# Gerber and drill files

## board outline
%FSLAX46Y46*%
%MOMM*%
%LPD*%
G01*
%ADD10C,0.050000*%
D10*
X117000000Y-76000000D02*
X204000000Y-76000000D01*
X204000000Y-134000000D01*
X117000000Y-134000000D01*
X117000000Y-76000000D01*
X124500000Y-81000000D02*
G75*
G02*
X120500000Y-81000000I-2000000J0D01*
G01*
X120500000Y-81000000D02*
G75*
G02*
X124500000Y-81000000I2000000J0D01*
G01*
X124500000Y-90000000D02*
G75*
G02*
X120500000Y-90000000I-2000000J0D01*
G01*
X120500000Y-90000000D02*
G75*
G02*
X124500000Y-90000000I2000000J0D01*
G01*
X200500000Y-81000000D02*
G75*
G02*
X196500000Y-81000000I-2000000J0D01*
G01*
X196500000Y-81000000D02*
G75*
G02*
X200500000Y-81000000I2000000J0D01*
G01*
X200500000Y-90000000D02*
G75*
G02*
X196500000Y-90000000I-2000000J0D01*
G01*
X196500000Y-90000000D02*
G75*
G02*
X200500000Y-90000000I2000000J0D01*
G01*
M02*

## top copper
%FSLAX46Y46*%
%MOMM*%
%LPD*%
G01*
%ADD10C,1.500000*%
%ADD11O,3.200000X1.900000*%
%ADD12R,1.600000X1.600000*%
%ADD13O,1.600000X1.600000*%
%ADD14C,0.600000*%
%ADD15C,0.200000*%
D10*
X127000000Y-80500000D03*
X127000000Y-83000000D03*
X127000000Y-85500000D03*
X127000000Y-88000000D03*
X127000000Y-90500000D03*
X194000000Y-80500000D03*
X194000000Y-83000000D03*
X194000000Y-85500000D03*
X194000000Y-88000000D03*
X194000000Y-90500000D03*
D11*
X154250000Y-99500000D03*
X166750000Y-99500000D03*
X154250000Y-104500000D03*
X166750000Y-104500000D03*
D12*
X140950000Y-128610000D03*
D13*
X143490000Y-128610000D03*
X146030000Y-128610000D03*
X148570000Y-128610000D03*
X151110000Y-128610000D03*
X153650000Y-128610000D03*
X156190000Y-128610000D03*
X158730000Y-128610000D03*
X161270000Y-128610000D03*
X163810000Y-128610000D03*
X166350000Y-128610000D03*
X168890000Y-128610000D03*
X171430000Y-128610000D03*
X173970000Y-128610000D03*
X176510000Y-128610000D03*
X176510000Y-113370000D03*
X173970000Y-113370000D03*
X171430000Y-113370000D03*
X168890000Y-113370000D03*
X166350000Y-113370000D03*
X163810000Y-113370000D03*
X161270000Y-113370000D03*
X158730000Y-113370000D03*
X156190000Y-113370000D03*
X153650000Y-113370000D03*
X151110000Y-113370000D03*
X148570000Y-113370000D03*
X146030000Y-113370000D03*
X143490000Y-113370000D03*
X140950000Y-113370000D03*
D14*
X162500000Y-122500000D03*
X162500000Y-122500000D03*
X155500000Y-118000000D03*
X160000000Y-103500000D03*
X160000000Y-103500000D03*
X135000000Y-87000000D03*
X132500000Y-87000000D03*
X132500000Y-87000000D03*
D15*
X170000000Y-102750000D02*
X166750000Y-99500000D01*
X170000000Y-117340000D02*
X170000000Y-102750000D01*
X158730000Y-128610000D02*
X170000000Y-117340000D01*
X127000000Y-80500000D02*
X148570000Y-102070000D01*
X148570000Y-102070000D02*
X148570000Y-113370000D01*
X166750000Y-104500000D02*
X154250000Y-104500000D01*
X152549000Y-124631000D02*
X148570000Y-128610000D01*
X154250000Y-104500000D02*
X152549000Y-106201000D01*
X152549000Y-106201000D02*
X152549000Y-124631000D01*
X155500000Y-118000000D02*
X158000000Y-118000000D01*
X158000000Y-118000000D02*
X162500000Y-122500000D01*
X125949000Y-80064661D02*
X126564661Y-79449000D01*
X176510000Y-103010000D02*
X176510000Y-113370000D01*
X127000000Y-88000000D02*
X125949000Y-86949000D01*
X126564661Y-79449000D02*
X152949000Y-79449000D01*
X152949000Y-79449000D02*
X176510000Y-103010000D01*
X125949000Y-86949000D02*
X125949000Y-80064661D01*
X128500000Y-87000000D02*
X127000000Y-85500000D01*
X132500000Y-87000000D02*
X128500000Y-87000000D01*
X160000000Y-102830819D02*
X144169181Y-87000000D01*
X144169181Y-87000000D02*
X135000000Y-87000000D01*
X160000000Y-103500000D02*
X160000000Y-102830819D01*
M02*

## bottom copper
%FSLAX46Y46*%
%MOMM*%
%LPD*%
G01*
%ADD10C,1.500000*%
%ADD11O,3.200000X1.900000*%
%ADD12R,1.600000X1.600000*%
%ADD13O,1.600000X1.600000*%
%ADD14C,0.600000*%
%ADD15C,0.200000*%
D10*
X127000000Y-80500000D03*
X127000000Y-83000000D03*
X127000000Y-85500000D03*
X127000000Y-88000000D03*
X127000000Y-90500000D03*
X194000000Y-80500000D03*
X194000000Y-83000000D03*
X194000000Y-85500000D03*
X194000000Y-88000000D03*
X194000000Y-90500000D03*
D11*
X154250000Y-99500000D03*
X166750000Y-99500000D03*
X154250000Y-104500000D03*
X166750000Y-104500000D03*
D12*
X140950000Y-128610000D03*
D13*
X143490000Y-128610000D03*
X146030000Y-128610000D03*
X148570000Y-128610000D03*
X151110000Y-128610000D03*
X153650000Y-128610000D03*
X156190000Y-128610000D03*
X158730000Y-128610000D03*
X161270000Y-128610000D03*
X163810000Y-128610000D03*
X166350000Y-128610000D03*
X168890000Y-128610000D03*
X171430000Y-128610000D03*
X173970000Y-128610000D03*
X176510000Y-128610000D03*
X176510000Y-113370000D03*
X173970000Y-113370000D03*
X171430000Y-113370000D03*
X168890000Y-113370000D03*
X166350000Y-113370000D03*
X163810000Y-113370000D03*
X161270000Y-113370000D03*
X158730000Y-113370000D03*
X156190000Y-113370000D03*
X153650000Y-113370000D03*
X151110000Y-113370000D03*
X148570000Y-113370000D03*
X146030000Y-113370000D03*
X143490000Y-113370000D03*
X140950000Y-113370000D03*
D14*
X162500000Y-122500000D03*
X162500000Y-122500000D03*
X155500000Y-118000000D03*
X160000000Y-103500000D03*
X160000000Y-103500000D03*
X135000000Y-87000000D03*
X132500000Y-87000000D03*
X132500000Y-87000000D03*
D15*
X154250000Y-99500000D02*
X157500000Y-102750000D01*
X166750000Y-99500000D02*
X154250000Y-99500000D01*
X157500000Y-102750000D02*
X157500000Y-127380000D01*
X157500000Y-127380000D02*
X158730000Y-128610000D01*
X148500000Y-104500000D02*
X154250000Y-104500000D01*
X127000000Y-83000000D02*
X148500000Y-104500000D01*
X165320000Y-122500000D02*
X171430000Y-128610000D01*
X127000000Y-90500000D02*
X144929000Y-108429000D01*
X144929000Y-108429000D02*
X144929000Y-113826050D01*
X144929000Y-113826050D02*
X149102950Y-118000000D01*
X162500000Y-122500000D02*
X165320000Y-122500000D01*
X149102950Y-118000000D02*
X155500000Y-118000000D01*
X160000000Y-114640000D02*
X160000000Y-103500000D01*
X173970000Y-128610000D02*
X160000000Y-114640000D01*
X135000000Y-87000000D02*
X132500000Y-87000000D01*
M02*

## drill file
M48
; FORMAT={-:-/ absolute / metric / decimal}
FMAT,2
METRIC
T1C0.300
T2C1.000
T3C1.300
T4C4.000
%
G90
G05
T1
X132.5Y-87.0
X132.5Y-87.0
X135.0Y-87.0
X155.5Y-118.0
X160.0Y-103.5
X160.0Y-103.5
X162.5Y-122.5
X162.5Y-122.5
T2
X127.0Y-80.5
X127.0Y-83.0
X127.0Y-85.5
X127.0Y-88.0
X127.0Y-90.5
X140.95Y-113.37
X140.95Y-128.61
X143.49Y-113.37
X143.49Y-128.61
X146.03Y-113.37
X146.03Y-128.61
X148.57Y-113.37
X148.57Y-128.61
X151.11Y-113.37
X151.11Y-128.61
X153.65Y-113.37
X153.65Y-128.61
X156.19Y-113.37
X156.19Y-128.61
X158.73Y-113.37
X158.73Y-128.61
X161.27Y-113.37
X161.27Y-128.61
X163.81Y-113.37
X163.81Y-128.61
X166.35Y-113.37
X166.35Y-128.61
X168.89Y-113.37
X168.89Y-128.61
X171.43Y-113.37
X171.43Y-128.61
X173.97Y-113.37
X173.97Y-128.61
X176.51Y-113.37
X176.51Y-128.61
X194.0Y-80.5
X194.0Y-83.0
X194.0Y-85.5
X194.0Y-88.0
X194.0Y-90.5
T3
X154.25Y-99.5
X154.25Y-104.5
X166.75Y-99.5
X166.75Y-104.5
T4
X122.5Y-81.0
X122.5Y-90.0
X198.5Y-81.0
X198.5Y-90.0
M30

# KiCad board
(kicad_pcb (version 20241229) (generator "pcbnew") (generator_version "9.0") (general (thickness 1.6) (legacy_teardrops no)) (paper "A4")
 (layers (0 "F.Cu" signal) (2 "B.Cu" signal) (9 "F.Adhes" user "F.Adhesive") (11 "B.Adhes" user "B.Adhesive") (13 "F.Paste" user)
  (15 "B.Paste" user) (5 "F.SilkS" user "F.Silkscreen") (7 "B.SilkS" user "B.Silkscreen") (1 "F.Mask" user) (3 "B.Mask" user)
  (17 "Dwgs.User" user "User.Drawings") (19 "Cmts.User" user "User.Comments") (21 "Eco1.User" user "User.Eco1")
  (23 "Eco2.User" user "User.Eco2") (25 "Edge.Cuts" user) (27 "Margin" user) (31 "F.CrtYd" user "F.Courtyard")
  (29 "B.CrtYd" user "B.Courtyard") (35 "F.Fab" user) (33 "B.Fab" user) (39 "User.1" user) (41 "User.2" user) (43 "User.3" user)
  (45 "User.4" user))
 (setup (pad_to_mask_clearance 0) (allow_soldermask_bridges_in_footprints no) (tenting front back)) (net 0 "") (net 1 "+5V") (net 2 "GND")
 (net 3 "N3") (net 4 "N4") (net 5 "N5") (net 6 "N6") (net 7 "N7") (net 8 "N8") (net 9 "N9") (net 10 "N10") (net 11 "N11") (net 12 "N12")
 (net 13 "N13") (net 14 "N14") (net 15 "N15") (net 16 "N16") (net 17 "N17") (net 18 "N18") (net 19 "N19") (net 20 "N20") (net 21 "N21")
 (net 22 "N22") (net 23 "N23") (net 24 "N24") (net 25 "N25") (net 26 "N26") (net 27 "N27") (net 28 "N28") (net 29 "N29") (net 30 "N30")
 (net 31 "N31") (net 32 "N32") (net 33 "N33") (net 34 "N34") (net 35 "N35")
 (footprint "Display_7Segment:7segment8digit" (layer "F.Cu") (at 160.5 85.5)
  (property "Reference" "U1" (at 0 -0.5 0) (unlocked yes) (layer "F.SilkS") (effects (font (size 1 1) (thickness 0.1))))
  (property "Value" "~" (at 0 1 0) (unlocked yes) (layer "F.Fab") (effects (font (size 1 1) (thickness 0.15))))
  (fp_circle (center -38 -4.5) (end -36 -4.5) (stroke (width 0.05) (type solid)) (fill no) (layer "Edge.Cuts"))
  (fp_circle (center -38 4.5) (end -36 4.5) (stroke (width 0.05) (type solid)) (fill no) (layer "Edge.Cuts"))
  (fp_circle (center 38 -4.5) (end 40 -4.5) (stroke (width 0.05) (type solid)) (fill no) (layer "Edge.Cuts"))
  (fp_circle (center 38 4.5) (end 40 4.5) (stroke (width 0.05) (type solid)) (fill no) (layer "Edge.Cuts"))
  (pad "" np_thru_hole circle (at -38 -4.5) (size 4 4) (drill 4) (layers "*.Cu" "*.Mask"))
  (pad "" np_thru_hole circle (at -38 4.5) (size 4 4) (drill 4) (layers "*.Cu" "*.Mask"))
  (pad "" np_thru_hole circle (at 38 -4.5) (size 4 4) (drill 4) (layers "*.Cu" "*.Mask"))
  (pad "" np_thru_hole circle (at 38 4.5) (size 4 4) (drill 4) (layers "*.Cu" "*.Mask"))
  (pad "1" thru_hole circle (at -33.5 -5) (size 1.5 1.5) (drill 1) (layers "*.Cu" "*.Mask") (remove_unused_layers no) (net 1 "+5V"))
  (pad "2" thru_hole circle (at -33.5 -2.5) (size 1.5 1.5) (drill 1) (layers "*.Cu" "*.Mask") (remove_unused_layers no) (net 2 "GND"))
  (pad "3" thru_hole circle (at -33.5 0) (size 1.5 1.5) (drill 1) (layers "*.Cu" "*.Mask") (remove_unused_layers no) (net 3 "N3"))
  (pad "4" thru_hole circle (at -33.5 2.5) (size 1.5 1.5) (drill 1) (layers "*.Cu" "*.Mask") (remove_unused_layers no) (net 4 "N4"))
  (pad "5" thru_hole circle (at -33.5 5) (size 1.5 1.5) (drill 1) (layers "*.Cu" "*.Mask") (remove_unused_layers no) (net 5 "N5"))
  (pad "6" thru_hole circle (at 33.5 -5) (size 1.5 1.5) (drill 1) (layers "*.Cu" "*.Mask") (remove_unused_layers no) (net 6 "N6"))
  (pad "7" thru_hole circle (at 33.5 -2.5) (size 1.5 1.5) (drill 1) (layers "*.Cu" "*.Mask") (remove_unused_layers no) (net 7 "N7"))
  (pad "8" thru_hole circle (at 33.5 0) (size 1.5 1.5) (drill 1) (layers "*.Cu" "*.Mask") (remove_unused_layers no) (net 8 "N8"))
  (pad "9" thru_hole circle (at 33.5 2.5) (size 1.5 1.5) (drill 1) (layers "*.Cu" "*.Mask") (remove_unused_layers no) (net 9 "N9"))
  (pad "10" thru_hole circle (at 33.5 5) (size 1.5 1.5) (drill 1) (layers "*.Cu" "*.Mask") (remove_unused_layers no) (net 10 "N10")))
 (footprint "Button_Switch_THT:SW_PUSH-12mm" (layer "F.Cu") (at 154.25 99.5)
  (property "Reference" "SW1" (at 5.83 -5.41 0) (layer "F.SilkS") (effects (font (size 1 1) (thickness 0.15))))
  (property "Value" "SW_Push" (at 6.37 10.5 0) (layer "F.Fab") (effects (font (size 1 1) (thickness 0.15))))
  (pad "1" thru_hole oval (at 0 0) (size 3.2 1.9) (drill 1.3) (layers "*.Cu" "*.Mask") (remove_unused_layers no) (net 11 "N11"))
  (pad "1" thru_hole oval (at 12.5 0) (size 3.2 1.9) (drill 1.3) (layers "*.Cu" "*.Mask") (remove_unused_layers no) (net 11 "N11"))
  (pad "2" thru_hole oval (at 0 5) (size 3.2 1.9) (drill 1.3) (layers "*.Cu" "*.Mask") (remove_unused_layers no) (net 2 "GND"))
  (pad "2" thru_hole oval (at 12.5 5) (size 3.2 1.9) (drill 1.3) (layers "*.Cu" "*.Mask") (remove_unused_layers no) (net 2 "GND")))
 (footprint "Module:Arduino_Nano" (layer "F.Cu") (at 140.95 128.61 90)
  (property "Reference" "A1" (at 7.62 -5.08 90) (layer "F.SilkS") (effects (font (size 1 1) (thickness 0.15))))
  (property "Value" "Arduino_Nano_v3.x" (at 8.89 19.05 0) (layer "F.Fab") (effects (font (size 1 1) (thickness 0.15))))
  (pad "1" thru_hole rect (at 0 0 90) (size 1.6 1.6) (drill 1) (layers "*.Cu" "*.Mask") (remove_unused_layers no) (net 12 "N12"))
  (pad "2" thru_hole oval (at 0 2.54 90) (size 1.6 1.6) (drill 1) (layers "*.Cu" "*.Mask") (remove_unused_layers no) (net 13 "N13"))
  (pad "3" thru_hole oval (at 0 5.08 90) (size 1.6 1.6) (drill 1) (layers "*.Cu" "*.Mask") (remove_unused_layers no) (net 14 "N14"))
  (pad "4" thru_hole oval (at 0 7.62 90) (size 1.6 1.6) (drill 1) (layers "*.Cu" "*.Mask") (remove_unused_layers no) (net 2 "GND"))
  (pad "5" thru_hole oval (at 0 10.16 90) (size 1.6 1.6) (drill 1) (layers "*.Cu" "*.Mask") (remove_unused_layers no) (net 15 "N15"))
  (pad "6" thru_hole oval (at 0 12.7 90) (size 1.6 1.6) (drill 1) (layers "*.Cu" "*.Mask") (remove_unused_layers no) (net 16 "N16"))
  (pad "7" thru_hole oval (at 0 15.24 90) (size 1.6 1.6) (drill 1) (layers "*.Cu" "*.Mask") (remove_unused_layers no) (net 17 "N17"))
  (pad "8" thru_hole oval (at 0 17.78 90) (size 1.6 1.6) (drill 1) (layers "*.Cu" "*.Mask") (remove_unused_layers no) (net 11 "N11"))
  (pad "9" thru_hole oval (at 0 20.32 90) (size 1.6 1.6) (drill 1) (layers "*.Cu" "*.Mask") (remove_unused_layers no) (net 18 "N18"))
  (pad "10" thru_hole oval (at 0 22.86 90) (size 1.6 1.6) (drill 1) (layers "*.Cu" "*.Mask") (remove_unused_layers no) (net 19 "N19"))
  (pad "11" thru_hole oval (at 0 25.4 90) (size 1.6 1.6) (drill 1) (layers "*.Cu" "*.Mask") (remove_unused_layers no) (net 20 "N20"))
  (pad "12" thru_hole oval (at 0 27.94 90) (size 1.6 1.6) (drill 1) (layers "*.Cu" "*.Mask") (remove_unused_layers no) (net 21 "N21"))
  (pad "13" thru_hole oval (at 0 30.48 90) (size 1.6 1.6) (drill 1) (layers "*.Cu" "*.Mask") (remove_unused_layers no) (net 5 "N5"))
  (pad "14" thru_hole oval (at 0 33.02 90) (size 1.6 1.6) (drill 1) (layers "*.Cu" "*.Mask") (remove_unused_layers no) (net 3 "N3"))
  (pad "15" thru_hole oval (at 0 35.56 90) (size 1.6 1.6) (drill 1) (layers "*.Cu" "*.Mask") (remove_unused_layers no) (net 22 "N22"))
  (pad "16" thru_hole oval (at 15.24 35.56 90) (size 1.6 1.6) (drill 1) (layers "*.Cu" "*.Mask") (remove_unused_layers no) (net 4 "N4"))
  (pad "17" thru_hole oval (at 15.24 33.02 90) (size 1.6 1.6) (drill 1) (layers "*.Cu" "*.Mask") (remove_unused_layers no) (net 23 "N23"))
  (pad "18" thru_hole oval (at 15.24 30.48 90) (size 1.6 1.6) (drill 1) (layers "*.Cu" "*.Mask") (remove_unused_layers no) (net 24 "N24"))
  (pad "19" thru_hole oval (at 15.24 27.94 90) (size 1.6 1.6) (drill 1) (layers "*.Cu" "*.Mask") (remove_unused_layers no) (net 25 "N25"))
  (pad "20" thru_hole oval (at 15.24 25.4 90) (size 1.6 1.6) (drill 1) (layers "*.Cu" "*.Mask") (remove_unused_layers no) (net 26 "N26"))
  (pad "21" thru_hole oval (at 15.24 22.86 90) (size 1.6 1.6) (drill 1) (layers "*.Cu" "*.Mask") (remove_unused_layers no) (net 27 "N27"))
  (pad "22" thru_hole oval (at 15.24 20.32 90) (size 1.6 1.6) (drill 1) (layers "*.Cu" "*.Mask") (remove_unused_layers no) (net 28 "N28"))
  (pad "23" thru_hole oval (at 15.24 17.78 90) (size 1.6 1.6) (drill 1) (layers "*.Cu" "*.Mask") (remove_unused_layers no) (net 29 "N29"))
  (pad "24" thru_hole oval (at 15.24 15.24 90) (size 1.6 1.6) (drill 1) (layers "*.Cu" "*.Mask") (remove_unused_layers no) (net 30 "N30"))
  (pad "25" thru_hole oval (at 15.24 12.7 90) (size 1.6 1.6) (drill 1) (layers "*.Cu" "*.Mask") (remove_unused_layers no) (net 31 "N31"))
  (pad "26" thru_hole oval (at 15.24 10.16 90) (size 1.6 1.6) (drill 1) (layers "*.Cu" "*.Mask") (remove_unused_layers no) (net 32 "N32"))
  (pad "27" thru_hole oval (at 15.24 7.62 90) (size 1.6 1.6) (drill 1) (layers "*.Cu" "*.Mask") (remove_unused_layers no) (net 1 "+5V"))
  (pad "28" thru_hole oval (at 15.24 5.08 90) (size 1.6 1.6) (drill 1) (layers "*.Cu" "*.Mask") (remove_unused_layers no) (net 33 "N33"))
  (pad "29" thru_hole oval (at 15.24 2.54 90) (size 1.6 1.6) (drill 1) (layers "*.Cu" "*.Mask") (remove_unused_layers no) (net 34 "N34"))
  (pad "30" thru_hole oval (at 15.24 0 90) (size 1.6 1.6) (drill 1) (layers "*.Cu" "*.Mask") (remove_unused_layers no) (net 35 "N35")))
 (gr_rect (start 117 76) (end 204 134) (stroke (width 0.05) (type default)) (fill no) (layer "Edge.Cuts"))
 (segment (start 170 102.75) (end 166.75 99.5) (width 0.2) (layer "F.Cu") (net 11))
 (segment (start 170 117.34) (end 170 102.75) (width 0.2) (layer "F.Cu") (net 11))
 (segment (start 158.73 128.61) (end 170 117.34) (width 0.2) (layer "F.Cu") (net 11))
 (segment (start 154.25 99.5) (end 157.5 102.75) (width 0.2) (layer "B.Cu") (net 11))
 (segment (start 166.75 99.5) (end 154.25 99.5) (width 0.2) (layer "B.Cu") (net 11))
 (segment (start 157.5 102.75) (end 157.5 127.38) (width 0.2) (layer "B.Cu") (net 11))
 (segment (start 157.5 127.38) (end 158.73 128.61) (width 0.2) (layer "B.Cu") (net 11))
 (segment (start 127 80.5) (end 148.57 102.07) (width 0.2) (layer "F.Cu") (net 1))
 (segment (start 148.57 102.07) (end 148.57 113.37) (width 0.2) (layer "F.Cu") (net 1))
 (segment (start 166.75 104.5) (end 154.25 104.5) (width 0.2) (layer "F.Cu") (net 2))
 (segment (start 152.549 124.631) (end 148.57 128.61) (width 0.2) (layer "F.Cu") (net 2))
 (segment (start 154.25 104.5) (end 152.549 106.201) (width 0.2) (layer "F.Cu") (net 2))
 (segment (start 152.549 106.201) (end 152.549 124.631) (width 0.2) (layer "F.Cu") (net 2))
 (segment (start 148.5 104.5) (end 154.25 104.5) (width 0.2) (layer "B.Cu") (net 2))
 (segment (start 127 83) (end 148.5 104.5) (width 0.2) (layer "B.Cu") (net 2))
 (segment (start 155.5 118) (end 158 118) (width 0.2) (layer "F.Cu") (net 5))
 (segment (start 158 118) (end 162.5 122.5) (width 0.2) (layer "F.Cu") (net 5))
 (via (at 162.5 122.5) (size 0.6) (drill 0.3) (layers "F.Cu" "B.Cu") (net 5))
 (via (at 162.5 122.5) (size 0.6) (drill 0.3) (layers "F.Cu" "B.Cu") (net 5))
 (via (at 155.5 118) (size 0.6) (drill 0.3) (layers "F.Cu" "B.Cu") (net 5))
 (segment (start 165.32 122.5) (end 171.43 128.61) (width 0.2) (layer "B.Cu") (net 5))
 (segment (start 127 90.5) (end 144.929 108.429) (width 0.2) (layer "B.Cu") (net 5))
 (segment (start 144.929 108.429) (end 144.929 113.82605) (width 0.2) (layer "B.Cu") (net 5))
 (segment (start 144.929 113.82605) (end 149.10295 118) (width 0.2) (layer "B.Cu") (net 5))
 (segment (start 162.5 122.5) (end 165.32 122.5) (width 0.2) (layer "B.Cu") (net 5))
 (segment (start 149.10295 118) (end 155.5 118) (width 0.2) (layer "B.Cu") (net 5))
 (segment (start 125.949 80.064661) (end 126.564661 79.449) (width 0.2) (layer "F.Cu") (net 4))
 (segment (start 176.51 103.01) (end 176.51 113.37) (width 0.2) (layer "F.Cu") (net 4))
 (segment (start 127 88) (end 125.949 86.949) (width 0.2) (layer "F.Cu") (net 4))
 (segment (start 126.564661 79.449) (end 152.949 79.449) (width 0.2) (layer "F.Cu") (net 4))
 (segment (start 152.949 79.449) (end 176.51 103.01) (width 0.2) (layer "F.Cu") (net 4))
 (segment (start 125.949 86.949) (end 125.949 80.064661) (width 0.2) (layer "F.Cu") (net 4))
 (segment (start 128.5 87) (end 127 85.5) (width 0.2) (layer "F.Cu") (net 3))
 (segment (start 132.5 87) (end 128.5 87) (width 0.2) (layer "F.Cu") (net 3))
 (segment (start 160 102.830819) (end 144.169181 87) (width 0.2) (layer "F.Cu") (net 3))
 (segment (start 144.169181 87) (end 135 87) (width 0.2) (layer "F.Cu") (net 3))
 (segment (start 160 103.5) (end 160 102.830819) (width 0.2) (layer "F.Cu") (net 3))
 (via (at 160 103.5) (size 0.6) (drill 0.3) (layers "F.Cu" "B.Cu") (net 3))
 (via (at 160 103.5) (size 0.6) (drill 0.3) (layers "F.Cu" "B.Cu") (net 3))
 (via (at 135 87) (size 0.6) (drill 0.3) (layers "F.Cu" "B.Cu") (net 3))
 (via (at 132.5 87) (size 0.6) (drill 0.3) (layers "F.Cu" "B.Cu") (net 3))
 (via (at 132.5 87) (size 0.6) (drill 0.3) (layers "F.Cu" "B.Cu") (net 3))
 (segment (start 160 114.64) (end 160 103.5) (width 0.2) (layer "B.Cu") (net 3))
 (segment (start 173.97 128.61) (end 160 114.64) (width 0.2) (layer "B.Cu") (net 3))
 (segment (start 135 87) (end 132.5 87) (width 0.2) (layer "B.Cu") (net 3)))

